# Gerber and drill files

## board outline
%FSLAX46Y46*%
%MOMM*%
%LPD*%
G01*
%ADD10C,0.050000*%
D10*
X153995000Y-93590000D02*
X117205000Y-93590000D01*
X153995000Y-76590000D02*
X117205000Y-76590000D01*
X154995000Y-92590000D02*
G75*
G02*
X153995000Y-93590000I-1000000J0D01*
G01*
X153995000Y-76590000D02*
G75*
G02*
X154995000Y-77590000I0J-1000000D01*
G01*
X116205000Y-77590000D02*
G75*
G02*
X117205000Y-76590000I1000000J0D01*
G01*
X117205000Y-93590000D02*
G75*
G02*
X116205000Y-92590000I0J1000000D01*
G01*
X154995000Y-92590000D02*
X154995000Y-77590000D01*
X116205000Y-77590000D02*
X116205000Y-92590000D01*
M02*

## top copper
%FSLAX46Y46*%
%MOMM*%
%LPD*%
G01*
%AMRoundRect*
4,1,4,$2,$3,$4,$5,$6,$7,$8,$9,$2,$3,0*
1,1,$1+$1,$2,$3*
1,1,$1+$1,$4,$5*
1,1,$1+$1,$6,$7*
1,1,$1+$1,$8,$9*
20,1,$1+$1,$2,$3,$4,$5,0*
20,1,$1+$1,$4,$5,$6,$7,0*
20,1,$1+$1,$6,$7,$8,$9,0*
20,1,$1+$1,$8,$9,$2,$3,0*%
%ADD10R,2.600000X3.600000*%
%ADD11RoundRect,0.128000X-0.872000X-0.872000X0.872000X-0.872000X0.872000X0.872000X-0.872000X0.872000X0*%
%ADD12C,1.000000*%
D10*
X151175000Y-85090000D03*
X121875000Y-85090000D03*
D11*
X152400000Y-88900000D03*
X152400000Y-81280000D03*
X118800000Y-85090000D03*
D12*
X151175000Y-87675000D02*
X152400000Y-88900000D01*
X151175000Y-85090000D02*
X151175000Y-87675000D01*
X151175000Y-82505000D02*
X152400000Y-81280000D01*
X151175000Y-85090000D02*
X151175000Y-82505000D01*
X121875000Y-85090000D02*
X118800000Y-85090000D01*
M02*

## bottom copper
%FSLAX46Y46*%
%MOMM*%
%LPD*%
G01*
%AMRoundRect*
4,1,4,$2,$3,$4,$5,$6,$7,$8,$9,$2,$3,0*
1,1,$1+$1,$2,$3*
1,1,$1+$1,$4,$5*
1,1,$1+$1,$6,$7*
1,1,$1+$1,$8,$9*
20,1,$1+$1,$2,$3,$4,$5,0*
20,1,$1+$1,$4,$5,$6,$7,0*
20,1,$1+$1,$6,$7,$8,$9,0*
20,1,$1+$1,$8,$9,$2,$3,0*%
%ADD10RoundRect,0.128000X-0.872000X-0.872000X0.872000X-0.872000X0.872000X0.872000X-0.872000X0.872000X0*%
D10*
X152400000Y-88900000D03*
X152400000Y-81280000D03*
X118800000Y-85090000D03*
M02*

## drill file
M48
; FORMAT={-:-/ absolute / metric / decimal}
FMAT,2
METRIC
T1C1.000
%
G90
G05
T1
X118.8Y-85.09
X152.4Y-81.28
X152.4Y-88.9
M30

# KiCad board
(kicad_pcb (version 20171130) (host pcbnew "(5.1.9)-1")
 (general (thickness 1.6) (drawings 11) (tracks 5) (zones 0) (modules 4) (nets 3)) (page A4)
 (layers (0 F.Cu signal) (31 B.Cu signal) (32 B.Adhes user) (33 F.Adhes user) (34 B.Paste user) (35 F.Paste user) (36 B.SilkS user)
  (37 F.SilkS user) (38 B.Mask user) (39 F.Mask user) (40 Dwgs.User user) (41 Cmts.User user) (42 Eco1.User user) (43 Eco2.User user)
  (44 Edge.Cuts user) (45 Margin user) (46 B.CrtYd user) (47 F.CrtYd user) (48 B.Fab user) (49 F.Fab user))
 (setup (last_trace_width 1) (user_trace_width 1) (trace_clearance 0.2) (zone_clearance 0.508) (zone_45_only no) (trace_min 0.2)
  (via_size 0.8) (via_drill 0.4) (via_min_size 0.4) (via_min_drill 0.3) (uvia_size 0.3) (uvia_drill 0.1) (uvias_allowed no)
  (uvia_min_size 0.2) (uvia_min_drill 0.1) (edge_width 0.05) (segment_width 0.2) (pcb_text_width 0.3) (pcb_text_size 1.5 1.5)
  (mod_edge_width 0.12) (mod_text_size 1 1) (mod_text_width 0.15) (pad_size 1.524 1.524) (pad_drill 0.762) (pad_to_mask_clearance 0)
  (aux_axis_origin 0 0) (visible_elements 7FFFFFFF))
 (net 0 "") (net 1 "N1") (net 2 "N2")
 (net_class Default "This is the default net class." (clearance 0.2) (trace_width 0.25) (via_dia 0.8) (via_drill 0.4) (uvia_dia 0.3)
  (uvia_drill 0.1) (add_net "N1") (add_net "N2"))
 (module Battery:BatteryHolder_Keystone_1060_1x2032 (layer F.Cu) (at 136.525 85.09 180)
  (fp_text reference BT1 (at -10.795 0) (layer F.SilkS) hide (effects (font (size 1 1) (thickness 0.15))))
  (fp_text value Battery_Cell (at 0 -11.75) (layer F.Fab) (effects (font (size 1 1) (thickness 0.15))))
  (pad 1 smd rect (at -14.65 0) (size 2.6 3.6) (layers F.Cu F.Paste F.Mask) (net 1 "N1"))
  (pad 2 smd rect (at 14.65 0) (size 2.6 3.6) (layers F.Cu F.Paste F.Mask) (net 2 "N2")))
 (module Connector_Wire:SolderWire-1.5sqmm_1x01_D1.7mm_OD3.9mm (layer F.Cu) (at 152.4 88.9)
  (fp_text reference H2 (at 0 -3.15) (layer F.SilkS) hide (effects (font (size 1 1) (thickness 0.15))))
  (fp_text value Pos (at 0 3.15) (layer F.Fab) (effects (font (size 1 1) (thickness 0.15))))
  (pad 1 thru_hole roundrect (at 0 0) (size 2 2) (drill 1) (layers *.Cu *.Mask) (roundrect_rratio 0.064) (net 1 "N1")))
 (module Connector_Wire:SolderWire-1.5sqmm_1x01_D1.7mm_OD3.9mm (layer F.Cu) (at 152.4 81.28)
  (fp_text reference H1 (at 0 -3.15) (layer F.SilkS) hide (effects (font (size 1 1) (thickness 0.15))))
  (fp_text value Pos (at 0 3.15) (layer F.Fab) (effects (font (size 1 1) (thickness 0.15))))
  (pad 1 thru_hole roundrect (at 0 0) (size 2 2) (drill 1) (layers *.Cu *.Mask) (roundrect_rratio 0.064) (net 1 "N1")))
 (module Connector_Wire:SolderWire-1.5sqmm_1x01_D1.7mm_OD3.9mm (layer F.Cu) (at 118.8 85.09)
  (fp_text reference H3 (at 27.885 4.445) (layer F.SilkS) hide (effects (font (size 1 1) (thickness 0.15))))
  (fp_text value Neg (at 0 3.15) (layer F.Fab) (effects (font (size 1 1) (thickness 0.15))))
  (pad 1 thru_hole roundrect (at 0 0) (size 2 2) (drill 1) (layers *.Cu *.Mask) (roundrect_rratio 0.064) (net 2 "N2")))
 (gr_line (start 153.995 93.59) (end 117.205 93.59) (layer Edge.Cuts) (width 0.05))
 (gr_line (start 153.995 76.59) (end 117.205 76.59) (layer Edge.Cuts) (width 0.05))
 (gr_arc (start 153.995 92.59) (end 153.995 93.59) (angle -90) (layer Edge.Cuts) (width 0.05))
 (gr_arc (start 153.995 77.59) (end 154.995 77.59) (angle -90) (layer Edge.Cuts) (width 0.05))
 (gr_arc (start 117.205 77.59) (end 117.205 76.59) (angle -90) (layer Edge.Cuts) (width 0.05))
 (gr_arc (start 117.205 92.59) (end 116.205 92.59) (angle -90) (layer Edge.Cuts) (width 0.05))
 (gr_line (start 154.995 92.59) (end 154.995 77.59) (layer Edge.Cuts) (width 0.05))
 (gr_line (start 116.205 77.59) (end 116.205 92.59) (layer Edge.Cuts) (width 0.05))
 (segment (start 151.175 87.675) (end 152.4 88.9) (width 1) (layer F.Cu) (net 1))
 (segment (start 151.175 85.09) (end 151.175 87.675) (width 1) (layer F.Cu) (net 1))
 (segment (start 151.175 82.505) (end 152.4 81.28) (width 1) (layer F.Cu) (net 1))
 (segment (start 151.175 85.09) (end 151.175 82.505) (width 1) (layer F.Cu) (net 1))
 (segment (start 121.875 85.09) (end 118.8 85.09) (width 1) (layer F.Cu) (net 2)))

